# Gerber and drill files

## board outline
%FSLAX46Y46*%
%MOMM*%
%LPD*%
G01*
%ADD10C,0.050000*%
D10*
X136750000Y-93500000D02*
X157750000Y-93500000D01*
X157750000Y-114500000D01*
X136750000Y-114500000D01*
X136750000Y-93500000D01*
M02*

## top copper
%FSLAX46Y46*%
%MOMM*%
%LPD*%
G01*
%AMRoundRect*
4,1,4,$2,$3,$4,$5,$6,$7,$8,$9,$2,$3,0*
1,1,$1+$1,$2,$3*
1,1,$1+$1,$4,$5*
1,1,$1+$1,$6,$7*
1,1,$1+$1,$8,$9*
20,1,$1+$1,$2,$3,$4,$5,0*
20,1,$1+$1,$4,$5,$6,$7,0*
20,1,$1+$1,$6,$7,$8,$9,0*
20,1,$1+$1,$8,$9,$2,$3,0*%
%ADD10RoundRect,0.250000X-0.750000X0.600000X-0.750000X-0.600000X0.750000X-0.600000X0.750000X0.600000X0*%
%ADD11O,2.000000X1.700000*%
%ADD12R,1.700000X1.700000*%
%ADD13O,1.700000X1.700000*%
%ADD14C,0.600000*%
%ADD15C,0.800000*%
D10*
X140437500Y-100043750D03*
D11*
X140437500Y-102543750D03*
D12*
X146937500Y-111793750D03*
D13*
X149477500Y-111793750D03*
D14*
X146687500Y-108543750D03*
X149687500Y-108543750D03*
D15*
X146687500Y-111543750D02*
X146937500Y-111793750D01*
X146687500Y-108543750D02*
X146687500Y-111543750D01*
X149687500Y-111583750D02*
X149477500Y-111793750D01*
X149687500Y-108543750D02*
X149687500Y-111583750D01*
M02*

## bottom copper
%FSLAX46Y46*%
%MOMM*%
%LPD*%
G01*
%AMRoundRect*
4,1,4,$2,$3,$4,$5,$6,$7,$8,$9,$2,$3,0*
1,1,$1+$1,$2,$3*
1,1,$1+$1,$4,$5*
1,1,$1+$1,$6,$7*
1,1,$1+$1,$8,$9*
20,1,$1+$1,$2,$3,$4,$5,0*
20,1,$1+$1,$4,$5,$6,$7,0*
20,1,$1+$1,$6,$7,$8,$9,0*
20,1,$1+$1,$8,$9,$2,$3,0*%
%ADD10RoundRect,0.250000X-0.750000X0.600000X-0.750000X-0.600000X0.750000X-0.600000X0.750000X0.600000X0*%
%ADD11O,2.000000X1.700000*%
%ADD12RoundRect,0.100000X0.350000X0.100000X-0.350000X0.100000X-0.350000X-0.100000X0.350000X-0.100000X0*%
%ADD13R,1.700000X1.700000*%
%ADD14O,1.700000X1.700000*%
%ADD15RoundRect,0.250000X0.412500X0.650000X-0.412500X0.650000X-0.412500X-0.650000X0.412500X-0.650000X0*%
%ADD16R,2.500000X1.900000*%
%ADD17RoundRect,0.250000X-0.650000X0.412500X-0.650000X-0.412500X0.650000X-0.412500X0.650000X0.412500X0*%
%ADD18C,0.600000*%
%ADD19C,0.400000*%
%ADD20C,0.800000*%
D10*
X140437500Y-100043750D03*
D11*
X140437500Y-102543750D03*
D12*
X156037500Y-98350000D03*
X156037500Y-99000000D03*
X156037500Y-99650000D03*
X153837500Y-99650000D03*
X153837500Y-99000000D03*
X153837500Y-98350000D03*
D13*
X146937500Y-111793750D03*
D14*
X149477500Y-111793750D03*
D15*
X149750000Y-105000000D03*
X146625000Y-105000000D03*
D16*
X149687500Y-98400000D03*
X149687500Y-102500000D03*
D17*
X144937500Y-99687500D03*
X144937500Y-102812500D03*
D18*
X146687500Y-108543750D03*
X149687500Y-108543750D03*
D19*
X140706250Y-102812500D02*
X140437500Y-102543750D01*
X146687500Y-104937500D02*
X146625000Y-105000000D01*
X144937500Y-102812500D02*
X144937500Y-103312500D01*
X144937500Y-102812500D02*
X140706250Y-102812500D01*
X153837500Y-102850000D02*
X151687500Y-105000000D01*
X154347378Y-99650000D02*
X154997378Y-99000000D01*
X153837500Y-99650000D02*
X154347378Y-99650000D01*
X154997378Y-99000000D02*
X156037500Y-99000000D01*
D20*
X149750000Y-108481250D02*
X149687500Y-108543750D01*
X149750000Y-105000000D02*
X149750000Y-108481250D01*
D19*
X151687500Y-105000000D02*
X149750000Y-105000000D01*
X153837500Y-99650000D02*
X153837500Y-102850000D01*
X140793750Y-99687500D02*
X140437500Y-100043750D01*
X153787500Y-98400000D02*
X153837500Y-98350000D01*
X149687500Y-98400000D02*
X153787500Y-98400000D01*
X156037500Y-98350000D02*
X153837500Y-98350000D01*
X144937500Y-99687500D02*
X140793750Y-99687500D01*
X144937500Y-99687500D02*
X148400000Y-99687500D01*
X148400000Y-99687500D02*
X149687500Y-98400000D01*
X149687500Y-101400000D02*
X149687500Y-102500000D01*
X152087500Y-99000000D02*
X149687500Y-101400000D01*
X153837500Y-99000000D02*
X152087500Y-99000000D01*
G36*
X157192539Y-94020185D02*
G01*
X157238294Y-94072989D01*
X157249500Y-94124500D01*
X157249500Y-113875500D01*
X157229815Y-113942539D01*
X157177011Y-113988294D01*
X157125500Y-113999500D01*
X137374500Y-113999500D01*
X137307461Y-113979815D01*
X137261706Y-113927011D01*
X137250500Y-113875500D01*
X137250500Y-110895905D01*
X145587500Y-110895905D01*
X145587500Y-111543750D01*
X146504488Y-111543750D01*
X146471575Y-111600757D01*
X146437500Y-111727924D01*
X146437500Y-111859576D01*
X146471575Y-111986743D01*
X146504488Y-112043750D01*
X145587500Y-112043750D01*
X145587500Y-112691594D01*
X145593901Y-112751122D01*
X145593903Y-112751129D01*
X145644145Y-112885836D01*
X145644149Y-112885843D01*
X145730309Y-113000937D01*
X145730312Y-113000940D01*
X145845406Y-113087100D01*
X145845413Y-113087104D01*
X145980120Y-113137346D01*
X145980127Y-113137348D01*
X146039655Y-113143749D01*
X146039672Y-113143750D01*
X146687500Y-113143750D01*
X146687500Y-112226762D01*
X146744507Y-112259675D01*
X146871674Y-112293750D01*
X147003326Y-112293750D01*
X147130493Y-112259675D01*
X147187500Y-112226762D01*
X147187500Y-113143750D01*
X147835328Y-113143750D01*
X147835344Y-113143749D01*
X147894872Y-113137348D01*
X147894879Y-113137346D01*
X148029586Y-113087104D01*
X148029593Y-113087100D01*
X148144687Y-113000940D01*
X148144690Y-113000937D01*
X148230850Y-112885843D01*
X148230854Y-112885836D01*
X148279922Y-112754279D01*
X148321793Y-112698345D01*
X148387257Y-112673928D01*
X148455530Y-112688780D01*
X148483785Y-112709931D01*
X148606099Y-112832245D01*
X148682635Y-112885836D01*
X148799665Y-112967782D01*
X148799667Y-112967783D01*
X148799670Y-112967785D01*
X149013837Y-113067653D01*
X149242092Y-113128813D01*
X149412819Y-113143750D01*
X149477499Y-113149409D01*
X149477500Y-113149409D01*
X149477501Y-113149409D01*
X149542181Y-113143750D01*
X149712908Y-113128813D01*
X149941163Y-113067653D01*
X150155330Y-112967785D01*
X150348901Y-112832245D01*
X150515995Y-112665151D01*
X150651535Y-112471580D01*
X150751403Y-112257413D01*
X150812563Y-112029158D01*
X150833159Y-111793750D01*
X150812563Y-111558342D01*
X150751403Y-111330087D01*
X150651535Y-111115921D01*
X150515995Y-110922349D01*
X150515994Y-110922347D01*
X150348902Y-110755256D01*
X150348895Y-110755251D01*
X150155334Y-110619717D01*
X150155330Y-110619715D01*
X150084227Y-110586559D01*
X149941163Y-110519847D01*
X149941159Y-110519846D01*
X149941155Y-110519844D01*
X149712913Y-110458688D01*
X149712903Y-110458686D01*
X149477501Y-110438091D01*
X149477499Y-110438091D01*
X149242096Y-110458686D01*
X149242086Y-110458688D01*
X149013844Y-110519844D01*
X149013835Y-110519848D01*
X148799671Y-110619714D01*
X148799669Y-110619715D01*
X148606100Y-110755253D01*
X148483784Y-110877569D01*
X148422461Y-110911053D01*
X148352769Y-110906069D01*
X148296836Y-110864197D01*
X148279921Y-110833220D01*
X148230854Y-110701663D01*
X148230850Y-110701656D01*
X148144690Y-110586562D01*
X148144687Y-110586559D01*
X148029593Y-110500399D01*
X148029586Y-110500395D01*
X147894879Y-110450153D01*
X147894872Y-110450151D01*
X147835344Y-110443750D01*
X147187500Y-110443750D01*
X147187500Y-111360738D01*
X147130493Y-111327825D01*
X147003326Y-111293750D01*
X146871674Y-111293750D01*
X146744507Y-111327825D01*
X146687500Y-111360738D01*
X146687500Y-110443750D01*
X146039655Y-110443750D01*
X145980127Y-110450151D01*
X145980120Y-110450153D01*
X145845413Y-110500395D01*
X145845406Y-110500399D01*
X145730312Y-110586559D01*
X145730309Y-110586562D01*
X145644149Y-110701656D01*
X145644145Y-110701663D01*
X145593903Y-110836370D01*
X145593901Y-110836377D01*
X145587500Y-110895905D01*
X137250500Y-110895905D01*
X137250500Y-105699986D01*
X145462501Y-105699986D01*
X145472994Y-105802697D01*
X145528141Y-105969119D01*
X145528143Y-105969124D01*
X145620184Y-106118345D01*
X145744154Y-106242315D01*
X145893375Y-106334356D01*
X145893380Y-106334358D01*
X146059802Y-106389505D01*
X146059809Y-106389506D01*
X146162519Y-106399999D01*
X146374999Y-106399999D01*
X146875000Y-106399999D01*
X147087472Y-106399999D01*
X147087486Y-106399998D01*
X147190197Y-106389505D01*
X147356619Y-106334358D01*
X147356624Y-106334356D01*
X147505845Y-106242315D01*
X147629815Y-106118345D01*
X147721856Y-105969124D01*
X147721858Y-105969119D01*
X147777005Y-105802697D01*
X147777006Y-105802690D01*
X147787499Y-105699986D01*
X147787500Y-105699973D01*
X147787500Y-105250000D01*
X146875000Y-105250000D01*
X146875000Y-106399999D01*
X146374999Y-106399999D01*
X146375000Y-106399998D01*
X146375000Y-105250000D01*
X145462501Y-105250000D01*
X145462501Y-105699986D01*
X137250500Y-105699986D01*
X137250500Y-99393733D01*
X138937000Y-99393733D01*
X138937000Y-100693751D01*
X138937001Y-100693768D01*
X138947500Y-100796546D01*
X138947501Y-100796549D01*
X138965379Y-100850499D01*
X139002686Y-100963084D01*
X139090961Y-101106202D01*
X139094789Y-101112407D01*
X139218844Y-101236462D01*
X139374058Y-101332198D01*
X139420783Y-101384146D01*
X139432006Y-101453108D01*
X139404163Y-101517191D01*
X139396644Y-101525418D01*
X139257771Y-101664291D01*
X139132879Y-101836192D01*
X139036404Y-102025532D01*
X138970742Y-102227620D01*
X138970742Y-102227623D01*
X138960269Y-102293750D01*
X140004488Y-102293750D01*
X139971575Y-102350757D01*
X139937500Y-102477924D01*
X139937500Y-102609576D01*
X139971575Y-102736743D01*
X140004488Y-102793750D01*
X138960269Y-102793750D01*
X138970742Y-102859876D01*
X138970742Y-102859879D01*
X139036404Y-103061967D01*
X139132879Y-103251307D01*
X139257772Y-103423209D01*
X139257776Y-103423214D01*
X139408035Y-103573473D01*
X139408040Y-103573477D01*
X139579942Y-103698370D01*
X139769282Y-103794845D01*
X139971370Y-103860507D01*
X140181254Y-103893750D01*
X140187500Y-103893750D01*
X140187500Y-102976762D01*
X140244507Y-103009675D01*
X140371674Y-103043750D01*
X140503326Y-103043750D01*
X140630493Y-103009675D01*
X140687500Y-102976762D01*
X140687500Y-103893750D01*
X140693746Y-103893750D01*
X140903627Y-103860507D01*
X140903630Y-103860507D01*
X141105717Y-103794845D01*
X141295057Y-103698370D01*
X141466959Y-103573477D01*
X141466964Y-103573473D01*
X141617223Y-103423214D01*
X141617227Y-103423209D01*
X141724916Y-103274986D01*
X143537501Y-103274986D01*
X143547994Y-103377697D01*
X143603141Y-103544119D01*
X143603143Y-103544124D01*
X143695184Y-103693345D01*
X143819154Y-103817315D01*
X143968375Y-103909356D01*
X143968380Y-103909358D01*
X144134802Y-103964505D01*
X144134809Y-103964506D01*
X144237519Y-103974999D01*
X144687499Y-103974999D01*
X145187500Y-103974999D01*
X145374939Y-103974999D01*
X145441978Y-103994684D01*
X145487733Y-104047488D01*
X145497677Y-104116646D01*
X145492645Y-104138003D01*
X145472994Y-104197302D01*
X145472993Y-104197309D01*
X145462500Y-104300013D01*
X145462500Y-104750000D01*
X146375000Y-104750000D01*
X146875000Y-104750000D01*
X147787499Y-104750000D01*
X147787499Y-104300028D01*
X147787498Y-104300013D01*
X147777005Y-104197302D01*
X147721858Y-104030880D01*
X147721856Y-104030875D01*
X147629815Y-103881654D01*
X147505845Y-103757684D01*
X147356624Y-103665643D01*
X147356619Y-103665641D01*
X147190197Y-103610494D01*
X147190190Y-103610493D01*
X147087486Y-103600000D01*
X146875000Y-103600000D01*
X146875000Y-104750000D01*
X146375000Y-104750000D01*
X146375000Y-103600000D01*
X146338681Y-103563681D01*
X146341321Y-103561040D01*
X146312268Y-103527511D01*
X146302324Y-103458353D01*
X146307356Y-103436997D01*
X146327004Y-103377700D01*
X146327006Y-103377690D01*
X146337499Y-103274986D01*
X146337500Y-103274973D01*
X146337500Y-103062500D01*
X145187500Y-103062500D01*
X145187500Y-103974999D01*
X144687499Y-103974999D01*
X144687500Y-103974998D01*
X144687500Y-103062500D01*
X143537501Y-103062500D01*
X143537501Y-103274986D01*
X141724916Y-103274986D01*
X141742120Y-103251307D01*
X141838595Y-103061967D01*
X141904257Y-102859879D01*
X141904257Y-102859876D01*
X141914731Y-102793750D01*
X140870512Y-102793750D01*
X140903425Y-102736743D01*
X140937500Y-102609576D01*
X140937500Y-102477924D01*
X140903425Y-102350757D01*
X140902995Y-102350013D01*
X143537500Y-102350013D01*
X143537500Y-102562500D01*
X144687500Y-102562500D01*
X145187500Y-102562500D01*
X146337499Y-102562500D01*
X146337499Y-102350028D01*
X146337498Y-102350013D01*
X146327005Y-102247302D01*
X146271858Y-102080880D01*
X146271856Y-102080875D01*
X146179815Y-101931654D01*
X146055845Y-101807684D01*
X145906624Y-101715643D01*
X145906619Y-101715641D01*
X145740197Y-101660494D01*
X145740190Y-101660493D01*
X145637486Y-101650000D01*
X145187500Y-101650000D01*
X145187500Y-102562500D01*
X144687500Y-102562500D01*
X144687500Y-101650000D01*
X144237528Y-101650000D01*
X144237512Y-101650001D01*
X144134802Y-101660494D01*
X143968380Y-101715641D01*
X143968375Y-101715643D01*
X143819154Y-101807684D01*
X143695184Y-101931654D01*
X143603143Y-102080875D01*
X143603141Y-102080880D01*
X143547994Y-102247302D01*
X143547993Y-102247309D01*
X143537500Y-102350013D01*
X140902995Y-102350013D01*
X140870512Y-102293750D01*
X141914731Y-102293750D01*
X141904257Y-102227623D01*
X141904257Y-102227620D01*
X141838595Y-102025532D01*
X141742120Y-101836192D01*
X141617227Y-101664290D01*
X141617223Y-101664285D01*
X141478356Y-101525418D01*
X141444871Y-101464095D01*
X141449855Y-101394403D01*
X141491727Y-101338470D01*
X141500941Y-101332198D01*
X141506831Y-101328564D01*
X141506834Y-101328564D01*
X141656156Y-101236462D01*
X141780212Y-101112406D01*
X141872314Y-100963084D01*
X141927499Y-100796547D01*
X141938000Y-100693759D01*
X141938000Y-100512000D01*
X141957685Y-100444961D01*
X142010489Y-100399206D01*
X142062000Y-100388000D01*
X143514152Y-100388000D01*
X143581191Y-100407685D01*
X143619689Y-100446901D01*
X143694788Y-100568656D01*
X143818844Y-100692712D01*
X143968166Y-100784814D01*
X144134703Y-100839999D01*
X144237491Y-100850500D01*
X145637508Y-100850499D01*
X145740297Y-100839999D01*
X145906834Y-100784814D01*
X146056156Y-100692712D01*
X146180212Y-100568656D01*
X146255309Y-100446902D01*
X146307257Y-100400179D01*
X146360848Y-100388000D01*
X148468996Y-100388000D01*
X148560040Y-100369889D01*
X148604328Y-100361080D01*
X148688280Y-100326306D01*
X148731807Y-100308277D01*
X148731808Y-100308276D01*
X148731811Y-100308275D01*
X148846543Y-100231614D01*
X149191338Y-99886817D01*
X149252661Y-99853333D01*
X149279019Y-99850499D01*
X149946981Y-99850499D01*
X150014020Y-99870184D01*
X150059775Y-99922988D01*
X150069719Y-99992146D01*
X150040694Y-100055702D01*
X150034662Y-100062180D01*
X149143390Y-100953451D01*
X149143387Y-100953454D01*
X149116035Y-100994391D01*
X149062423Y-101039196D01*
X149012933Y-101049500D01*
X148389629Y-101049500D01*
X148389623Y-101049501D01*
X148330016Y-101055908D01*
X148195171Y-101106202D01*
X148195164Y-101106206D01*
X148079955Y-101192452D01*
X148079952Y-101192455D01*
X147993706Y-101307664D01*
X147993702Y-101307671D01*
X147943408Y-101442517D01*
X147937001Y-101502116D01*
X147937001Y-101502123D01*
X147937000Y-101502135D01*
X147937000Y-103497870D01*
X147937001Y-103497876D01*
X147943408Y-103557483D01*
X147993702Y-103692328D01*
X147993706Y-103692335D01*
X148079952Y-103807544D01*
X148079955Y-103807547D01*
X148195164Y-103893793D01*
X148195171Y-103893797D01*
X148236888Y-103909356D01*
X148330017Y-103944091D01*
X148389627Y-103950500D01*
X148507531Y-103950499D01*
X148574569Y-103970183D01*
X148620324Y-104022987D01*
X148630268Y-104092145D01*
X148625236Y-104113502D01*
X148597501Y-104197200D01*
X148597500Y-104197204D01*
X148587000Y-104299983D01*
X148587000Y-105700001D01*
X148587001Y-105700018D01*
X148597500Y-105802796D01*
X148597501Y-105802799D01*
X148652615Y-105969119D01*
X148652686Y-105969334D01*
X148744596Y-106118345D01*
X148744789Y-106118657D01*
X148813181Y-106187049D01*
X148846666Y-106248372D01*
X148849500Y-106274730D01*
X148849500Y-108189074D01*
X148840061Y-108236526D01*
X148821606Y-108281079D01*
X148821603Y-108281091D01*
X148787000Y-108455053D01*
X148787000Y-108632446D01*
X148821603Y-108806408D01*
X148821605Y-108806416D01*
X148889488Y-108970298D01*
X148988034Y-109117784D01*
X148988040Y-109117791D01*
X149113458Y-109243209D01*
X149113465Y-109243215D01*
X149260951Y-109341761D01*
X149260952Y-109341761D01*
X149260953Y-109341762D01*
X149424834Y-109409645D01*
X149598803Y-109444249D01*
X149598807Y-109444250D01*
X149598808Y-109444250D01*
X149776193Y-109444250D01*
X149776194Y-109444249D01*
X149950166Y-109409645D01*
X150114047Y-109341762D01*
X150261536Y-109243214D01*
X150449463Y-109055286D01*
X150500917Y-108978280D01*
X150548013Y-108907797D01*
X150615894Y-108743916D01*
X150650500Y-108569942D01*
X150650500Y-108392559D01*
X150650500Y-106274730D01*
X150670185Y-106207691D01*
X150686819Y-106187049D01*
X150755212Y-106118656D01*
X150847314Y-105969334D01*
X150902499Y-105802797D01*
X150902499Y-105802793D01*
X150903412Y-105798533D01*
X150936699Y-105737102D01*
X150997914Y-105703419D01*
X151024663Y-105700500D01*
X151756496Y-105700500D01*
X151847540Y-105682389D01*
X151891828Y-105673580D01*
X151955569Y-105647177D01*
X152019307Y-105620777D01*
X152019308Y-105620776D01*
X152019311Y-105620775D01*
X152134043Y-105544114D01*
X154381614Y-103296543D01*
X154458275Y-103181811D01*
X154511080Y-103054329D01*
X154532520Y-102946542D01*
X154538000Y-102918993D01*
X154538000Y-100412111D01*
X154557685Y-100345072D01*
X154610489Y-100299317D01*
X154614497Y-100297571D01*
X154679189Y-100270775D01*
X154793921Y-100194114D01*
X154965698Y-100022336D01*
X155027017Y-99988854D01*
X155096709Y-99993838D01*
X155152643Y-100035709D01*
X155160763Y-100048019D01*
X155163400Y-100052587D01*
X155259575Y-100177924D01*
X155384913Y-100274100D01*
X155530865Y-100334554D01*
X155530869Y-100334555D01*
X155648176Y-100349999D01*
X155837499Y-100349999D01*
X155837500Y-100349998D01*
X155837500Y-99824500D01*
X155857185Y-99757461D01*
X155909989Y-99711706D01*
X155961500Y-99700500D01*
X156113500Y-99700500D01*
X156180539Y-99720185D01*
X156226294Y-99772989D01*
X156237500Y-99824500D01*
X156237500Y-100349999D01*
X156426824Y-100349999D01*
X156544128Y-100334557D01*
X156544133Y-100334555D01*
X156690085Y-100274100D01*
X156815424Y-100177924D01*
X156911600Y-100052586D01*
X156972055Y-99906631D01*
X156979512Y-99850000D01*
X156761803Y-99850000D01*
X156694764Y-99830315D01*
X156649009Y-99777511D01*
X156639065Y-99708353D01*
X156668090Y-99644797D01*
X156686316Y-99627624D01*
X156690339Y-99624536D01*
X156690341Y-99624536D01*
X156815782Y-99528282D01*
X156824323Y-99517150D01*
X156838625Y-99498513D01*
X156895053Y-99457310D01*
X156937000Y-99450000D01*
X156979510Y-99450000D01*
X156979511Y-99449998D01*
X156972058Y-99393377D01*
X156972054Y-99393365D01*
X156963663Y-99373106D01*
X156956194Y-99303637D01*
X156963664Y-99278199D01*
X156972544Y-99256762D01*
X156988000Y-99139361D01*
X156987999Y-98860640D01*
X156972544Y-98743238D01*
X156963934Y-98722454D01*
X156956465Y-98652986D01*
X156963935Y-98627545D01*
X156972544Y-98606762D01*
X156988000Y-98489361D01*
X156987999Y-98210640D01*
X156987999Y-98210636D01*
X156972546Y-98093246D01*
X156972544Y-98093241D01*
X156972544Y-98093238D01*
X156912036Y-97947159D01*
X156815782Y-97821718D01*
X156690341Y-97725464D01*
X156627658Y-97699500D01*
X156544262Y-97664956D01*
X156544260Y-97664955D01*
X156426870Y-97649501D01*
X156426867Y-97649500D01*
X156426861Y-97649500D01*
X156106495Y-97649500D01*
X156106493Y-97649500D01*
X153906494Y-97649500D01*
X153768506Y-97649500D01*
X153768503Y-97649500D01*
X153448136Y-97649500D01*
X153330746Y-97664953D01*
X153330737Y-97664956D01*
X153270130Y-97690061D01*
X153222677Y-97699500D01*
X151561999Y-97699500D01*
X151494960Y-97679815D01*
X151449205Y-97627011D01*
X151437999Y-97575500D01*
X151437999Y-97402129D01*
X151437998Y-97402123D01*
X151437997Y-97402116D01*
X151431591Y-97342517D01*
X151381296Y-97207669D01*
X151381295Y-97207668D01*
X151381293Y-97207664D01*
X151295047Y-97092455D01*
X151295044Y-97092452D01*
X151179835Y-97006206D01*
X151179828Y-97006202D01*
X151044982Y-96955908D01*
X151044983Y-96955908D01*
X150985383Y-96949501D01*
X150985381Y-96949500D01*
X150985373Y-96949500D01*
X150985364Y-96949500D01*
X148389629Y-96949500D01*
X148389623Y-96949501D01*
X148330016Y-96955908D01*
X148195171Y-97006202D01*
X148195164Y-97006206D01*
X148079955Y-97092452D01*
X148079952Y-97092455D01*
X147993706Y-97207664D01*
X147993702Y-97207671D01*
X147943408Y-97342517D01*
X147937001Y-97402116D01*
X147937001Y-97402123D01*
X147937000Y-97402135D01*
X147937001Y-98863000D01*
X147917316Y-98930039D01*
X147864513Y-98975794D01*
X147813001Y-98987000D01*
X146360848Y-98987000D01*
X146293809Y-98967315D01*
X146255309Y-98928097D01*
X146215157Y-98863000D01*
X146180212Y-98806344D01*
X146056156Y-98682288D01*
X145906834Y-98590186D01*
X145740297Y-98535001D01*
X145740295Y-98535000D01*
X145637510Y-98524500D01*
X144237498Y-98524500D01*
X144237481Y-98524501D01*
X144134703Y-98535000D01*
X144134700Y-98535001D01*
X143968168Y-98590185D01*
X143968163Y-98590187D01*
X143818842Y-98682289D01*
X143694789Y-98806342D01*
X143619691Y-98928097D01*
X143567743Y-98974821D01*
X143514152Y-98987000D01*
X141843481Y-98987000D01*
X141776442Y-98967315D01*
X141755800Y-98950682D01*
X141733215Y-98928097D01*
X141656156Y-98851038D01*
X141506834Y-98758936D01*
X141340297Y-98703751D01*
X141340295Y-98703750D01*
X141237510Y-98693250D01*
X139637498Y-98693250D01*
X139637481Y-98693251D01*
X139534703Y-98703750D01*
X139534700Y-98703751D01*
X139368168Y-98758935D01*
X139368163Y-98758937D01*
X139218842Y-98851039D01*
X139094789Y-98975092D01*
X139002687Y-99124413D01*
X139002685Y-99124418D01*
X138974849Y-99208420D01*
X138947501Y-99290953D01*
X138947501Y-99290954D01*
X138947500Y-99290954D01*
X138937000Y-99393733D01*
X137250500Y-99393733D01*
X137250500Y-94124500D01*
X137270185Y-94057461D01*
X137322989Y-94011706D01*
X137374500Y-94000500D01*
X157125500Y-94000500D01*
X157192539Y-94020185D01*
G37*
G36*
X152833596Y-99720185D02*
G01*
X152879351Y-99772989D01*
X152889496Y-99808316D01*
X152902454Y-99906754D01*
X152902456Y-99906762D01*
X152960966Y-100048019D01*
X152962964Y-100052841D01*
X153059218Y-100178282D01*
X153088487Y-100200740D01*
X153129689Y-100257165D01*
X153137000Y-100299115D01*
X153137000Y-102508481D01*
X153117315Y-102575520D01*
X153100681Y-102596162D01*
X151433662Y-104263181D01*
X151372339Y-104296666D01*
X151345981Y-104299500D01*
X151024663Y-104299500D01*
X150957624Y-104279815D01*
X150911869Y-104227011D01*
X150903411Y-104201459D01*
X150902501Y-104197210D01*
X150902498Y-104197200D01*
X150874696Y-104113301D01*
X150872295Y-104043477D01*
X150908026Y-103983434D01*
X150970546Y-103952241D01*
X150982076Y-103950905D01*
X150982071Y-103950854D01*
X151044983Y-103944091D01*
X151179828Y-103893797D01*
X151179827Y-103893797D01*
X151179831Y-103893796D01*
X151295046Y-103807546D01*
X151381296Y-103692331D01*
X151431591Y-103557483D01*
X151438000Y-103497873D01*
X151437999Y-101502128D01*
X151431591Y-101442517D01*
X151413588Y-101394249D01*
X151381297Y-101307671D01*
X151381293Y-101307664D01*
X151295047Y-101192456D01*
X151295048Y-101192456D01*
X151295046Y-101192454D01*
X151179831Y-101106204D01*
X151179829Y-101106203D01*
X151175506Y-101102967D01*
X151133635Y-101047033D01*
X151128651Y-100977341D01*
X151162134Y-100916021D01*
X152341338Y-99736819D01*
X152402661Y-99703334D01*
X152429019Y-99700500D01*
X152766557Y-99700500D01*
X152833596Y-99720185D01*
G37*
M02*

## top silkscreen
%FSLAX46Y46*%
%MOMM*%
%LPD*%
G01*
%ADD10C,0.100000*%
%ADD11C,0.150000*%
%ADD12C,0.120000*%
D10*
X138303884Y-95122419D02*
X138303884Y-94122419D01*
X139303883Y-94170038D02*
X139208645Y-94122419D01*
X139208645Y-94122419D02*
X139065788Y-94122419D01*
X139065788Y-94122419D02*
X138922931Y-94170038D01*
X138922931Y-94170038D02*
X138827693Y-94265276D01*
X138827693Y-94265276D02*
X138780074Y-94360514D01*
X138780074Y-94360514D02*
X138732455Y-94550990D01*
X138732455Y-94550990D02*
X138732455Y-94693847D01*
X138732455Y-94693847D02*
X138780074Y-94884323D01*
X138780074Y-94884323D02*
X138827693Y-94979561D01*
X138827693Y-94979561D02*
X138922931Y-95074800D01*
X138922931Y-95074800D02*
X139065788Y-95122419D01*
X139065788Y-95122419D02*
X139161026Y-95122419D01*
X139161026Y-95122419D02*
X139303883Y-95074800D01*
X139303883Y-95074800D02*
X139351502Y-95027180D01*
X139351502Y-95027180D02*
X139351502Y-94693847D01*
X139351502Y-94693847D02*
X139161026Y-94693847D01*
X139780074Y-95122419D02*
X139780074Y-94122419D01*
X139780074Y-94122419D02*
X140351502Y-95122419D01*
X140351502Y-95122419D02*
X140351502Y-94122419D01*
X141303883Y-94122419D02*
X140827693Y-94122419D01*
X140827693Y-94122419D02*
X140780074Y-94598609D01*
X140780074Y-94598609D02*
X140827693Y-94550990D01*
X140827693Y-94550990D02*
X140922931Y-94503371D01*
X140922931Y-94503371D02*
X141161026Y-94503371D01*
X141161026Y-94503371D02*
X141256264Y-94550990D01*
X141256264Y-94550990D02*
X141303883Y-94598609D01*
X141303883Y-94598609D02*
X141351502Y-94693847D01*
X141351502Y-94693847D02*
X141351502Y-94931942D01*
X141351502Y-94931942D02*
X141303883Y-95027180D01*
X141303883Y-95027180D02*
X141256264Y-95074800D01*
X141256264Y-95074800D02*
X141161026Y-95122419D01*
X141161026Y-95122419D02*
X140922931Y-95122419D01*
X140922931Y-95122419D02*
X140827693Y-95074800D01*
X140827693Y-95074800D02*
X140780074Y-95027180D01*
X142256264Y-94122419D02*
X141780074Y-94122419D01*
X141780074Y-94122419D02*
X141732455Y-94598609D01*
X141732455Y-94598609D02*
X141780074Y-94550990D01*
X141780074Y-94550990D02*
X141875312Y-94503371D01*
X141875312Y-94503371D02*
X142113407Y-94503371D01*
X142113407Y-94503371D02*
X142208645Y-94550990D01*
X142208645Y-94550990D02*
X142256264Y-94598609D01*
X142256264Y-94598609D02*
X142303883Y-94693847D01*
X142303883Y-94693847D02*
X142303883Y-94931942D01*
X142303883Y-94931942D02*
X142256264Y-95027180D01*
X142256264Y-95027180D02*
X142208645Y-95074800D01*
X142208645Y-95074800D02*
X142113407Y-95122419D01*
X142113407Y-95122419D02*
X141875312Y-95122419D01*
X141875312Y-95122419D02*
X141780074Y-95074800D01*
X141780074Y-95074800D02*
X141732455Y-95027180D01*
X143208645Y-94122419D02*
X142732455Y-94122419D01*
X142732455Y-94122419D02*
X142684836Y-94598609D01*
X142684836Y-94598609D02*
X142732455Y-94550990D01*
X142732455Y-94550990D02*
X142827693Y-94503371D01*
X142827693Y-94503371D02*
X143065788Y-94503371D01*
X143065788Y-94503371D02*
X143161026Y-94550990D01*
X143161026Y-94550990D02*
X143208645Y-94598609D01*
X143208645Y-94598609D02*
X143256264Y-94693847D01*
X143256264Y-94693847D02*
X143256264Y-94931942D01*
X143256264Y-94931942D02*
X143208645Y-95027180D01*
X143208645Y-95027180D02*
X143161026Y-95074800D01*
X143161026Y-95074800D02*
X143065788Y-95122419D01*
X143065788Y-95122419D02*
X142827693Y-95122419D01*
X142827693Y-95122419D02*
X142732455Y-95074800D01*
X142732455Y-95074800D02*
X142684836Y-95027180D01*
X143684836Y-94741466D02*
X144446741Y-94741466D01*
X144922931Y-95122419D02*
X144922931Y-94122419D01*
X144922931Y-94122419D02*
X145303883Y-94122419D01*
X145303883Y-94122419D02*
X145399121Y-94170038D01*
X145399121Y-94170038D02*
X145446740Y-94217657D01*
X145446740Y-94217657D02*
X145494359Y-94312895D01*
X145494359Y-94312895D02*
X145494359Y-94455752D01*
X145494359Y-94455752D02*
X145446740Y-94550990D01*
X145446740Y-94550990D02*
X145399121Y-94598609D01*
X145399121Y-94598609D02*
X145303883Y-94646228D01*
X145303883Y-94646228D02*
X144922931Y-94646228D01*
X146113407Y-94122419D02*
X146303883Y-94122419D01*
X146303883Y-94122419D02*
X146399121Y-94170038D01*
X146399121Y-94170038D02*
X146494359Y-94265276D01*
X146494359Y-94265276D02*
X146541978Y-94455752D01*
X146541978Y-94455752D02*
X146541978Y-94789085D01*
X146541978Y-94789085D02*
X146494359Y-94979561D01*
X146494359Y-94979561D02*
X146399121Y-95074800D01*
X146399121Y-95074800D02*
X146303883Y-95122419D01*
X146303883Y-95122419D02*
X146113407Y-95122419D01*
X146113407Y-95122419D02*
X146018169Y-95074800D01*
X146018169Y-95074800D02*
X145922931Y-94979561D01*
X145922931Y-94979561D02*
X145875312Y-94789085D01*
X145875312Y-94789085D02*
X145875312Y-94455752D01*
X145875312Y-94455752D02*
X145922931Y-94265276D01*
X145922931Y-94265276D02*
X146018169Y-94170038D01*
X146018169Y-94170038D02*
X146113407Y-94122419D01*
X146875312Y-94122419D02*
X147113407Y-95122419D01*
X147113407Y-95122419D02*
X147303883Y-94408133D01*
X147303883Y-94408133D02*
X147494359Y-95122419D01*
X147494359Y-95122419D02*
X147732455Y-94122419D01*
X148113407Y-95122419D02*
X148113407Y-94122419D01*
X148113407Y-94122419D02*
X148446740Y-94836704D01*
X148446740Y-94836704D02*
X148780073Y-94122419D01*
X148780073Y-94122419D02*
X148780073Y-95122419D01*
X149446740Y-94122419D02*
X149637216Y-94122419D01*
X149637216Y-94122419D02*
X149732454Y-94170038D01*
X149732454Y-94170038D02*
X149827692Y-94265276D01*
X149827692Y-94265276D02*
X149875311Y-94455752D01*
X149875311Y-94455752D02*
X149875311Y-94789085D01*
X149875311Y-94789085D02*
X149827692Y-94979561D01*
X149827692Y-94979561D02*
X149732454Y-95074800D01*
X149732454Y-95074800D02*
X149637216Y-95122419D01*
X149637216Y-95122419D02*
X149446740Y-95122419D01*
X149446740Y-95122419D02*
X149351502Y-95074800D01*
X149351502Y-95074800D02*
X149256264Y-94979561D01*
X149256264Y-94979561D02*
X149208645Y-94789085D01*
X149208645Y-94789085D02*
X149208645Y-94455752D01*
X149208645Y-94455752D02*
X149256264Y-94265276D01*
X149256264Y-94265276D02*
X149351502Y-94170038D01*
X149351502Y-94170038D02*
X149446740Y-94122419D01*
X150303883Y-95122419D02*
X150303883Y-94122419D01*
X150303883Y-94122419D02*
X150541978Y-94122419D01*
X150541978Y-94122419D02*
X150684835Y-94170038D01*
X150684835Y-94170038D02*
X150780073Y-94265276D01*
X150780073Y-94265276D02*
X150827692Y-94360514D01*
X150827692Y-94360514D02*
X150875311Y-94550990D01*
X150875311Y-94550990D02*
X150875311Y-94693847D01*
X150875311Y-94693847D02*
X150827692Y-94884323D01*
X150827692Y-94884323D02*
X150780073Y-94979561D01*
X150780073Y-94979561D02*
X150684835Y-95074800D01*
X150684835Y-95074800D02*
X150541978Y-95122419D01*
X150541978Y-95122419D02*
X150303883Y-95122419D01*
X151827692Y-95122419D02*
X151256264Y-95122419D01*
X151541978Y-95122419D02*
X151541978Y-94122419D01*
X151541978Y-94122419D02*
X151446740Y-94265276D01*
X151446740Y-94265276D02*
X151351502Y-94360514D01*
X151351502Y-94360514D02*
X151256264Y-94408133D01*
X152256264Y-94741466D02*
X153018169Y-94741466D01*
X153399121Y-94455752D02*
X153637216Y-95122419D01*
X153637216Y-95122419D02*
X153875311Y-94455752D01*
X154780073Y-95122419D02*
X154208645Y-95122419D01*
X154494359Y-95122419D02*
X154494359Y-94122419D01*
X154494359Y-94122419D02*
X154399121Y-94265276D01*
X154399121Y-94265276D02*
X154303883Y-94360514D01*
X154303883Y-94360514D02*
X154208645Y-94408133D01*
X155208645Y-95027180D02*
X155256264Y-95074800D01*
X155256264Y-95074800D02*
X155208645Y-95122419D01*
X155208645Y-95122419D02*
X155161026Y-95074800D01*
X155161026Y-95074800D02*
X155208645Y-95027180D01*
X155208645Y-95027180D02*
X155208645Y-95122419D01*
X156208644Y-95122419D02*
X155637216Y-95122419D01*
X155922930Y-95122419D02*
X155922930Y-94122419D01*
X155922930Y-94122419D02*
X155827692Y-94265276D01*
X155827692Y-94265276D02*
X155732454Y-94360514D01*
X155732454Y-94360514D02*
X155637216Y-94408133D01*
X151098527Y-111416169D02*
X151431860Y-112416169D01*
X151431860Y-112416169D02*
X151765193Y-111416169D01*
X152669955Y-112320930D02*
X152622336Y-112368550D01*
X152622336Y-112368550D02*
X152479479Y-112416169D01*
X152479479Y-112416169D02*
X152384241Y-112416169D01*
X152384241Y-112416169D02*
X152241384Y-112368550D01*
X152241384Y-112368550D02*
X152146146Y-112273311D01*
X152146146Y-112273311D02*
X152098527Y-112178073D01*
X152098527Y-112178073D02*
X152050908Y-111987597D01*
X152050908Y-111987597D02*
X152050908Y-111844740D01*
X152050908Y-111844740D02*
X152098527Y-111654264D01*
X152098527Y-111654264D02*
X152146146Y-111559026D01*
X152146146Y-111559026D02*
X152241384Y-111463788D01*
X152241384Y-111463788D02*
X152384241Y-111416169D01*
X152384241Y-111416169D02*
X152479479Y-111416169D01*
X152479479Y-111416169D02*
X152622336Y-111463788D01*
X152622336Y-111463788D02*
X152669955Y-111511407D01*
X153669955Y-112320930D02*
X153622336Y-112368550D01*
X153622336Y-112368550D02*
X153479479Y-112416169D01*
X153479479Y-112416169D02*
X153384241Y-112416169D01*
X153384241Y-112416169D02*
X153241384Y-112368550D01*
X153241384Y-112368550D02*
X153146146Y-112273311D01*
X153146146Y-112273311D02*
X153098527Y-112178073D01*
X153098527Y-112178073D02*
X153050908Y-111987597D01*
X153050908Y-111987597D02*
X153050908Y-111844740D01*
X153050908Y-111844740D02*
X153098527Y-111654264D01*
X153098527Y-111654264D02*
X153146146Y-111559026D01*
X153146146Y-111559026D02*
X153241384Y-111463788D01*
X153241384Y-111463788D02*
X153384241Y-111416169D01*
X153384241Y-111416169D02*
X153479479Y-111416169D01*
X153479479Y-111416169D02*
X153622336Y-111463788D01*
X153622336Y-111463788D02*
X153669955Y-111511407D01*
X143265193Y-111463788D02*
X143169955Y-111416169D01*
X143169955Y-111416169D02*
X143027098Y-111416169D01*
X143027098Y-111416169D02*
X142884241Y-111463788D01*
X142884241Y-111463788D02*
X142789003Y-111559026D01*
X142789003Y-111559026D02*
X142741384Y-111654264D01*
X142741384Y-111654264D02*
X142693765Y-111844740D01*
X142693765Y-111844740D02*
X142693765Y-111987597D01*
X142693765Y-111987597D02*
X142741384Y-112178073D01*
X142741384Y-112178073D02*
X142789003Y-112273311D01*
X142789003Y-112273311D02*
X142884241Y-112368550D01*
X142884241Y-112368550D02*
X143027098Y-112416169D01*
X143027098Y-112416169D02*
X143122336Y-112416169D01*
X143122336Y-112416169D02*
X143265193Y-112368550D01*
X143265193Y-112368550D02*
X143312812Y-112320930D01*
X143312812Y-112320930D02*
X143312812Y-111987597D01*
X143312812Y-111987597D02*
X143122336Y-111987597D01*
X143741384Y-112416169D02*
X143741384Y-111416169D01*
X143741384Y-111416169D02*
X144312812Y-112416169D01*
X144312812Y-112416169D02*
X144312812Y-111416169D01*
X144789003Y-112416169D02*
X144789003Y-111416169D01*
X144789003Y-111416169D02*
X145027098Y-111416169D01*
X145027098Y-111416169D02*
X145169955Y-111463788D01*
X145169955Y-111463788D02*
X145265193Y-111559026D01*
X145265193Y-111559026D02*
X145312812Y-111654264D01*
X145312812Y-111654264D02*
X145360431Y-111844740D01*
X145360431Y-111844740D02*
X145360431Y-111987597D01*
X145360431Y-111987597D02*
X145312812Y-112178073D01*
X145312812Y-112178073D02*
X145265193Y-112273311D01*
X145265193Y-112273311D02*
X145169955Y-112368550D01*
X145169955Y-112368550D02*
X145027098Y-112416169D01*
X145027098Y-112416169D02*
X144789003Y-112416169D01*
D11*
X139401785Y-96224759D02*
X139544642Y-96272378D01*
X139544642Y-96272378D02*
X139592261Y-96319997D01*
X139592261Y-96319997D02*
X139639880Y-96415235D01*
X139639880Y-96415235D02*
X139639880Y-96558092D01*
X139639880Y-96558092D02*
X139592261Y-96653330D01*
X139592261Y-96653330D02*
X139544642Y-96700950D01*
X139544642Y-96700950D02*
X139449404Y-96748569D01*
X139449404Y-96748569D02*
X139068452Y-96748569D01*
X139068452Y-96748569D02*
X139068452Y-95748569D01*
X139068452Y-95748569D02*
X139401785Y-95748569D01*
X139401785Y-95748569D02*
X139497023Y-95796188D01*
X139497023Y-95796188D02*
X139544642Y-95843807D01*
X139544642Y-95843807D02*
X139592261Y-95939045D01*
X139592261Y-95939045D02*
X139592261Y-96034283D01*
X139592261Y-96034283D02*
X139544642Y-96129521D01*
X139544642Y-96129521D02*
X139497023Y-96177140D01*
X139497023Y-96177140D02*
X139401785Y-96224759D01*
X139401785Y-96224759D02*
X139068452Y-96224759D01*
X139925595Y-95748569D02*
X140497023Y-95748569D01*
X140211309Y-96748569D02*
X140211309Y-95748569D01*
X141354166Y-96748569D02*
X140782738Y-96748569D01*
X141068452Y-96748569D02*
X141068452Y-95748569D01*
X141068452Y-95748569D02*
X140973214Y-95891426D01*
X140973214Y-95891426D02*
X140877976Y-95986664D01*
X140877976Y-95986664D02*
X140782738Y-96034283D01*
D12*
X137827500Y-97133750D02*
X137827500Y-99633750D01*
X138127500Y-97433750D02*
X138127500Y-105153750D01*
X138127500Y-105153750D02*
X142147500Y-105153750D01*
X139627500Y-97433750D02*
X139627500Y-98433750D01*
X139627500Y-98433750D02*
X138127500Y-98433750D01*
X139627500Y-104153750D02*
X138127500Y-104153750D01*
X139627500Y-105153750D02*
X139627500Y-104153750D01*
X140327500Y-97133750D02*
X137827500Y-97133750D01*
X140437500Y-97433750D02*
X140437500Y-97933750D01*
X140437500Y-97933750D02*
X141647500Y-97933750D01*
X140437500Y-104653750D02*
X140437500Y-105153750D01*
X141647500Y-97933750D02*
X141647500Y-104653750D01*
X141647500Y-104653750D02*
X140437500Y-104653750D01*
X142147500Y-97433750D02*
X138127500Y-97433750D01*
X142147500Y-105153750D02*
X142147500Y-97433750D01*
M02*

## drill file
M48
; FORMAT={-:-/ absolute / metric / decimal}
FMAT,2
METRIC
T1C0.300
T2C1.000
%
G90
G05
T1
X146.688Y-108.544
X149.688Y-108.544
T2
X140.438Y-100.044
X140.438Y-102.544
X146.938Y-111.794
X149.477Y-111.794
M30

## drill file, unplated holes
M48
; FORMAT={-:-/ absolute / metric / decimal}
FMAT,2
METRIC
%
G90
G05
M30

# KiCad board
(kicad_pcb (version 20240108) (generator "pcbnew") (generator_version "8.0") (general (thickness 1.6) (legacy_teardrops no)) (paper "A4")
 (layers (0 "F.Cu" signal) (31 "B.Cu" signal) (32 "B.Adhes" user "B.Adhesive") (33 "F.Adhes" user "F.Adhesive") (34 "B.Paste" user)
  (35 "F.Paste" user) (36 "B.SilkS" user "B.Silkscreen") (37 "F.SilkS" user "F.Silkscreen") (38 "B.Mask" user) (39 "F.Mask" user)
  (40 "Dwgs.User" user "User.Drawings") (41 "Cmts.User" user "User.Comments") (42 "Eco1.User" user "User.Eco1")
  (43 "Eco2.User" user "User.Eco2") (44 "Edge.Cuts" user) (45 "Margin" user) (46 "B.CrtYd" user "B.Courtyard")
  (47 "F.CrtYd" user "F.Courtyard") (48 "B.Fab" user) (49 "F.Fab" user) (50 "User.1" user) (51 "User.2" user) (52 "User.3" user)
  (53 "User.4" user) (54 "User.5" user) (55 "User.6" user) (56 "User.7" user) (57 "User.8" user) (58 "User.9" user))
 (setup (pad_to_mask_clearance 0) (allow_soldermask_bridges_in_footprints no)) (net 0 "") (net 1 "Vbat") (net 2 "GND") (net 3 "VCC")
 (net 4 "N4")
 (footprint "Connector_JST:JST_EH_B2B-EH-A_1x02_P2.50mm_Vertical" (layer "F.Cu") (at 140.4375 100.04375 -90)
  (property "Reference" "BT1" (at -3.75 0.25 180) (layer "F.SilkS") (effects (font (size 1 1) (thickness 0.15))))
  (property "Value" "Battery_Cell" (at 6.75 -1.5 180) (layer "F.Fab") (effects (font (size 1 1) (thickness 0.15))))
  (fp_line (start -2.91 2.61) (end -0.41 2.61) (stroke (width 0.12) (type solid)) (layer "F.SilkS"))
  (fp_line (start -2.61 2.31) (end 5.11 2.31) (stroke (width 0.12) (type solid)) (layer "F.SilkS"))
  (fp_line (start 5.11 2.31) (end 5.11 -1.71) (stroke (width 0.12) (type solid)) (layer "F.SilkS"))
  (fp_line (start -2.61 0.81) (end -1.61 0.81) (stroke (width 0.12) (type solid)) (layer "F.SilkS"))
  (fp_line (start -1.61 0.81) (end -1.61 2.31) (stroke (width 0.12) (type solid)) (layer "F.SilkS"))
  (fp_line (start 4.11 0.81) (end 4.11 2.31) (stroke (width 0.12) (type solid)) (layer "F.SilkS"))
  (fp_line (start 5.11 0.81) (end 4.11 0.81) (stroke (width 0.12) (type solid)) (layer "F.SilkS"))
  (fp_line (start -2.91 0.11) (end -2.91 2.61) (stroke (width 0.12) (type solid)) (layer "F.SilkS"))
  (fp_line (start -2.61 0) (end -2.11 0) (stroke (width 0.12) (type solid)) (layer "F.SilkS"))
  (fp_line (start -2.11 0) (end -2.11 -1.21) (stroke (width 0.12) (type solid)) (layer "F.SilkS"))
  (fp_line (start 4.61 0) (end 5.11 0) (stroke (width 0.12) (type solid)) (layer "F.SilkS"))
  (fp_line (start -2.11 -1.21) (end 4.61 -1.21) (stroke (width 0.12) (type solid)) (layer "F.SilkS"))
  (fp_line (start 4.61 -1.21) (end 4.61 0) (stroke (width 0.12) (type solid)) (layer "F.SilkS"))
  (fp_line (start -2.61 -1.71) (end -2.61 2.31) (stroke (width 0.12) (type solid)) (layer "F.SilkS"))
  (fp_line (start 5.11 -1.71) (end -2.61 -1.71) (stroke (width 0.12) (type solid)) (layer "F.SilkS"))
  (pad "1" thru_hole roundrect (at 0 0 270) (size 1.7 2) (drill 1) (layers "*.Cu" "*.Mask") (remove_unused_layers no)
   (roundrect_rratio 0.147059) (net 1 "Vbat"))
  (pad "2" thru_hole oval (at 2.5 0 270) (size 1.7 2) (drill 1) (layers "*.Cu" "*.Mask") (remove_unused_layers no) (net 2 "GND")))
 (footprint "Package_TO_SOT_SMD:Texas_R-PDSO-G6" (layer "B.Cu") (at 154.9375 99 180)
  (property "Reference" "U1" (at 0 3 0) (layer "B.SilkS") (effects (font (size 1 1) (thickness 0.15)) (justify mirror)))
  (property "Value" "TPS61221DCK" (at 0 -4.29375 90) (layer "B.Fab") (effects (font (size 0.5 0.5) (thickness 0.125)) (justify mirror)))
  (pad "1" smd roundrect (at -1.1 0.65 180) (size 0.9 0.4) (layers "B.Cu" "B.Paste" "B.Mask") (roundrect_rratio 0.25) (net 1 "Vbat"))
  (pad "2" smd roundrect (at -1.1 0 180) (size 0.9 0.4) (layers "B.Cu" "B.Paste" "B.Mask") (roundrect_rratio 0.25) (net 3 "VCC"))
  (pad "3" smd roundrect (at -1.1 -0.65 180) (size 0.9 0.4) (layers "B.Cu" "B.Paste" "B.Mask") (roundrect_rratio 0.25) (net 2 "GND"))
  (pad "4" smd roundrect (at 1.1 -0.65 180) (size 0.9 0.4) (layers "B.Cu" "B.Paste" "B.Mask") (roundrect_rratio 0.25) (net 3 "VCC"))
  (pad "5" smd roundrect (at 1.1 0 180) (size 0.9 0.4) (layers "B.Cu" "B.Paste" "B.Mask") (roundrect_rratio 0.25) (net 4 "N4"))
  (pad "6" smd roundrect (at 1.1 0.65 180) (size 0.9 0.4) (layers "B.Cu" "B.Paste" "B.Mask") (roundrect_rratio 0.25) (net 1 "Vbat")))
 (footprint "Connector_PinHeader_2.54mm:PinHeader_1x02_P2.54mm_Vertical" (layer "B.Cu") (at 146.9375 111.79375 -90)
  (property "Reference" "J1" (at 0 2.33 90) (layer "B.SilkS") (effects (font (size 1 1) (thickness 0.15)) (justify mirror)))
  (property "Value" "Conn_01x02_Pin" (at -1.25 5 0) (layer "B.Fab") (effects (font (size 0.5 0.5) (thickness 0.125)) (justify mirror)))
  (pad "1" thru_hole rect (at 0 0 270) (size 1.7 1.7) (drill 1) (layers "*.Cu" "*.Mask") (remove_unused_layers no) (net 2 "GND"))
  (pad "2" thru_hole oval (at 0 -2.54 270) (size 1.7 1.7) (drill 1) (layers "*.Cu" "*.Mask") (remove_unused_layers no) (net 3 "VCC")))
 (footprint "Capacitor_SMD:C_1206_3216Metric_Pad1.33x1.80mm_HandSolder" (layer "B.Cu") (at 148.1875 105 180)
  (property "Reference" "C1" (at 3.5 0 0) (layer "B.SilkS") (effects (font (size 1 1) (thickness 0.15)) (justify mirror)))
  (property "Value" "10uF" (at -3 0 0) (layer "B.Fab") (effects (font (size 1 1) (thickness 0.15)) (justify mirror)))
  (pad "1" smd roundrect (at -1.5625 0 180) (size 1.325 1.8) (layers "B.Cu" "B.Paste" "B.Mask") (roundrect_rratio 0.188679) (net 3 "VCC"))
  (pad "2" smd roundrect (at 1.5625 0 180) (size 1.325 1.8) (layers "B.Cu" "B.Paste" "B.Mask") (roundrect_rratio 0.188679) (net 2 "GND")))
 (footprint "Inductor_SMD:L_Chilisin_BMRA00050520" (layer "B.Cu") (at 149.6875 100.45 -90)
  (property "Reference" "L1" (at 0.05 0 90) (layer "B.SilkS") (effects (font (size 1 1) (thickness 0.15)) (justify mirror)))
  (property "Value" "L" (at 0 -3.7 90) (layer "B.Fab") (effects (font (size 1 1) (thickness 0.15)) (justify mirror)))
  (pad "1" smd rect (at -2.05 0 270) (size 1.9 2.5) (layers "B.Cu" "B.Paste" "B.Mask") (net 1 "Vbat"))
  (pad "2" smd rect (at 2.05 0 270) (size 1.9 2.5) (layers "B.Cu" "B.Paste" "B.Mask") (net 4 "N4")))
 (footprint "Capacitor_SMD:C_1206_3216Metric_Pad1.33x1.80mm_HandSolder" (layer "B.Cu") (at 144.9375 101.25 -90)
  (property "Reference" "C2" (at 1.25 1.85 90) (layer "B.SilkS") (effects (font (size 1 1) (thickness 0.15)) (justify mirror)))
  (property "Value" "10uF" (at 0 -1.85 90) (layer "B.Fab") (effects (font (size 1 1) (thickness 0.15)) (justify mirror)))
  (pad "1" smd roundrect (at -1.5625 0 270) (size 1.325 1.8) (layers "B.Cu" "B.Paste" "B.Mask") (roundrect_rratio 0.188679) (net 1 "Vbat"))
  (pad "2" smd roundrect (at 1.5625 0 270) (size 1.325 1.8) (layers "B.Cu" "B.Paste" "B.Mask") (roundrect_rratio 0.188679) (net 2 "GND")))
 (gr_rect (start 136.75 93.5) (end 157.75 114.5) (stroke (width 0.05) (type default)) (fill none) (layer "Edge.Cuts"))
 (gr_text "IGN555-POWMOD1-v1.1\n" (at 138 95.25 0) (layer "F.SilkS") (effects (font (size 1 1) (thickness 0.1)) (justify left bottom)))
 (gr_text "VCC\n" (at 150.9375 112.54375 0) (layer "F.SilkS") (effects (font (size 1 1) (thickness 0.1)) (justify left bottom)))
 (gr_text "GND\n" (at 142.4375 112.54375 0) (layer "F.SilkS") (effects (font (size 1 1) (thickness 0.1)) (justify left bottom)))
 (segment (start 146.6875 111.54375) (end 146.9375 111.79375) (width 0.8) (layer "F.Cu") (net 2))
 (segment (start 146.6875 108.54375) (end 146.6875 111.54375) (width 0.8) (layer "F.Cu") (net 2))
 (via (at 146.6875 108.54375) (size 0.6) (drill 0.3) (layers "F.Cu" "B.Cu") (free yes) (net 2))
 (segment (start 140.70625 102.8125) (end 140.4375 102.54375) (width 0.4) (layer "B.Cu") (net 2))
 (segment (start 146.6875 104.9375) (end 146.625 105) (width 0.4) (layer "B.Cu") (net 2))
 (segment (start 144.9375 102.8125) (end 144.9375 103.3125) (width 0.4) (layer "B.Cu") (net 2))
 (segment (start 144.9375 102.8125) (end 140.70625 102.8125) (width 0.4) (layer "B.Cu") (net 2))
 (segment (start 149.6875 111.58375) (end 149.4775 111.79375) (width 0.8) (layer "F.Cu") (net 3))
 (segment (start 149.6875 108.54375) (end 149.6875 111.58375) (width 0.8) (layer "F.Cu") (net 3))
 (via (at 149.6875 108.54375) (size 0.6) (drill 0.3) (layers "F.Cu" "B.Cu") (free yes) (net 3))
 (segment (start 153.8375 102.85) (end 151.6875 105) (width 0.4) (layer "B.Cu") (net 3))
 (segment (start 154.347378 99.65) (end 154.997378 99) (width 0.4) (layer "B.Cu") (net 3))
 (segment (start 153.8375 99.65) (end 154.347378 99.65) (width 0.4) (layer "B.Cu") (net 3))
 (segment (start 154.997378 99) (end 156.0375 99) (width 0.4) (layer "B.Cu") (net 3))
 (segment (start 149.75 108.48125) (end 149.6875 108.54375) (width 0.8) (layer "B.Cu") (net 3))
 (segment (start 149.75 105) (end 149.75 108.48125) (width 0.8) (layer "B.Cu") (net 3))
 (segment (start 151.6875 105) (end 149.75 105) (width 0.4) (layer "B.Cu") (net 3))
 (segment (start 153.8375 99.65) (end 153.8375 102.85) (width 0.4) (layer "B.Cu") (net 3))
 (segment (start 140.79375 99.6875) (end 140.4375 100.04375) (width 0.4) (layer "B.Cu") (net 1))
 (segment (start 153.7875 98.4) (end 153.8375 98.35) (width 0.4) (layer "B.Cu") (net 1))
 (segment (start 149.6875 98.4) (end 153.7875 98.4) (width 0.4) (layer "B.Cu") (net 1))
 (segment (start 156.0375 98.35) (end 153.8375 98.35) (width 0.4) (layer "B.Cu") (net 1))
 (segment (start 144.9375 99.6875) (end 140.79375 99.6875) (width 0.4) (layer "B.Cu") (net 1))
 (segment (start 144.9375 99.6875) (end 148.4 99.6875) (width 0.4) (layer "B.Cu") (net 1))
 (segment (start 148.4 99.6875) (end 149.6875 98.4) (width 0.4) (layer "B.Cu") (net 1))
 (segment (start 149.6875 101.4) (end 149.6875 102.5) (width 0.4) (layer "B.Cu") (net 4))
 (segment (start 152.0875 99) (end 149.6875 101.4) (width 0.4) (layer "B.Cu") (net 4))
 (segment (start 153.8375 99) (end 152.0875 99) (width 0.4) (layer "B.Cu") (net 4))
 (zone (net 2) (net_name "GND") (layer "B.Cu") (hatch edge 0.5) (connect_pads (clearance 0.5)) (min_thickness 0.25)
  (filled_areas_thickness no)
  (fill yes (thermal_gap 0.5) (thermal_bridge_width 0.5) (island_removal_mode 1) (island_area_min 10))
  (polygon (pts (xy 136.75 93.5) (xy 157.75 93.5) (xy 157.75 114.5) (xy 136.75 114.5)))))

